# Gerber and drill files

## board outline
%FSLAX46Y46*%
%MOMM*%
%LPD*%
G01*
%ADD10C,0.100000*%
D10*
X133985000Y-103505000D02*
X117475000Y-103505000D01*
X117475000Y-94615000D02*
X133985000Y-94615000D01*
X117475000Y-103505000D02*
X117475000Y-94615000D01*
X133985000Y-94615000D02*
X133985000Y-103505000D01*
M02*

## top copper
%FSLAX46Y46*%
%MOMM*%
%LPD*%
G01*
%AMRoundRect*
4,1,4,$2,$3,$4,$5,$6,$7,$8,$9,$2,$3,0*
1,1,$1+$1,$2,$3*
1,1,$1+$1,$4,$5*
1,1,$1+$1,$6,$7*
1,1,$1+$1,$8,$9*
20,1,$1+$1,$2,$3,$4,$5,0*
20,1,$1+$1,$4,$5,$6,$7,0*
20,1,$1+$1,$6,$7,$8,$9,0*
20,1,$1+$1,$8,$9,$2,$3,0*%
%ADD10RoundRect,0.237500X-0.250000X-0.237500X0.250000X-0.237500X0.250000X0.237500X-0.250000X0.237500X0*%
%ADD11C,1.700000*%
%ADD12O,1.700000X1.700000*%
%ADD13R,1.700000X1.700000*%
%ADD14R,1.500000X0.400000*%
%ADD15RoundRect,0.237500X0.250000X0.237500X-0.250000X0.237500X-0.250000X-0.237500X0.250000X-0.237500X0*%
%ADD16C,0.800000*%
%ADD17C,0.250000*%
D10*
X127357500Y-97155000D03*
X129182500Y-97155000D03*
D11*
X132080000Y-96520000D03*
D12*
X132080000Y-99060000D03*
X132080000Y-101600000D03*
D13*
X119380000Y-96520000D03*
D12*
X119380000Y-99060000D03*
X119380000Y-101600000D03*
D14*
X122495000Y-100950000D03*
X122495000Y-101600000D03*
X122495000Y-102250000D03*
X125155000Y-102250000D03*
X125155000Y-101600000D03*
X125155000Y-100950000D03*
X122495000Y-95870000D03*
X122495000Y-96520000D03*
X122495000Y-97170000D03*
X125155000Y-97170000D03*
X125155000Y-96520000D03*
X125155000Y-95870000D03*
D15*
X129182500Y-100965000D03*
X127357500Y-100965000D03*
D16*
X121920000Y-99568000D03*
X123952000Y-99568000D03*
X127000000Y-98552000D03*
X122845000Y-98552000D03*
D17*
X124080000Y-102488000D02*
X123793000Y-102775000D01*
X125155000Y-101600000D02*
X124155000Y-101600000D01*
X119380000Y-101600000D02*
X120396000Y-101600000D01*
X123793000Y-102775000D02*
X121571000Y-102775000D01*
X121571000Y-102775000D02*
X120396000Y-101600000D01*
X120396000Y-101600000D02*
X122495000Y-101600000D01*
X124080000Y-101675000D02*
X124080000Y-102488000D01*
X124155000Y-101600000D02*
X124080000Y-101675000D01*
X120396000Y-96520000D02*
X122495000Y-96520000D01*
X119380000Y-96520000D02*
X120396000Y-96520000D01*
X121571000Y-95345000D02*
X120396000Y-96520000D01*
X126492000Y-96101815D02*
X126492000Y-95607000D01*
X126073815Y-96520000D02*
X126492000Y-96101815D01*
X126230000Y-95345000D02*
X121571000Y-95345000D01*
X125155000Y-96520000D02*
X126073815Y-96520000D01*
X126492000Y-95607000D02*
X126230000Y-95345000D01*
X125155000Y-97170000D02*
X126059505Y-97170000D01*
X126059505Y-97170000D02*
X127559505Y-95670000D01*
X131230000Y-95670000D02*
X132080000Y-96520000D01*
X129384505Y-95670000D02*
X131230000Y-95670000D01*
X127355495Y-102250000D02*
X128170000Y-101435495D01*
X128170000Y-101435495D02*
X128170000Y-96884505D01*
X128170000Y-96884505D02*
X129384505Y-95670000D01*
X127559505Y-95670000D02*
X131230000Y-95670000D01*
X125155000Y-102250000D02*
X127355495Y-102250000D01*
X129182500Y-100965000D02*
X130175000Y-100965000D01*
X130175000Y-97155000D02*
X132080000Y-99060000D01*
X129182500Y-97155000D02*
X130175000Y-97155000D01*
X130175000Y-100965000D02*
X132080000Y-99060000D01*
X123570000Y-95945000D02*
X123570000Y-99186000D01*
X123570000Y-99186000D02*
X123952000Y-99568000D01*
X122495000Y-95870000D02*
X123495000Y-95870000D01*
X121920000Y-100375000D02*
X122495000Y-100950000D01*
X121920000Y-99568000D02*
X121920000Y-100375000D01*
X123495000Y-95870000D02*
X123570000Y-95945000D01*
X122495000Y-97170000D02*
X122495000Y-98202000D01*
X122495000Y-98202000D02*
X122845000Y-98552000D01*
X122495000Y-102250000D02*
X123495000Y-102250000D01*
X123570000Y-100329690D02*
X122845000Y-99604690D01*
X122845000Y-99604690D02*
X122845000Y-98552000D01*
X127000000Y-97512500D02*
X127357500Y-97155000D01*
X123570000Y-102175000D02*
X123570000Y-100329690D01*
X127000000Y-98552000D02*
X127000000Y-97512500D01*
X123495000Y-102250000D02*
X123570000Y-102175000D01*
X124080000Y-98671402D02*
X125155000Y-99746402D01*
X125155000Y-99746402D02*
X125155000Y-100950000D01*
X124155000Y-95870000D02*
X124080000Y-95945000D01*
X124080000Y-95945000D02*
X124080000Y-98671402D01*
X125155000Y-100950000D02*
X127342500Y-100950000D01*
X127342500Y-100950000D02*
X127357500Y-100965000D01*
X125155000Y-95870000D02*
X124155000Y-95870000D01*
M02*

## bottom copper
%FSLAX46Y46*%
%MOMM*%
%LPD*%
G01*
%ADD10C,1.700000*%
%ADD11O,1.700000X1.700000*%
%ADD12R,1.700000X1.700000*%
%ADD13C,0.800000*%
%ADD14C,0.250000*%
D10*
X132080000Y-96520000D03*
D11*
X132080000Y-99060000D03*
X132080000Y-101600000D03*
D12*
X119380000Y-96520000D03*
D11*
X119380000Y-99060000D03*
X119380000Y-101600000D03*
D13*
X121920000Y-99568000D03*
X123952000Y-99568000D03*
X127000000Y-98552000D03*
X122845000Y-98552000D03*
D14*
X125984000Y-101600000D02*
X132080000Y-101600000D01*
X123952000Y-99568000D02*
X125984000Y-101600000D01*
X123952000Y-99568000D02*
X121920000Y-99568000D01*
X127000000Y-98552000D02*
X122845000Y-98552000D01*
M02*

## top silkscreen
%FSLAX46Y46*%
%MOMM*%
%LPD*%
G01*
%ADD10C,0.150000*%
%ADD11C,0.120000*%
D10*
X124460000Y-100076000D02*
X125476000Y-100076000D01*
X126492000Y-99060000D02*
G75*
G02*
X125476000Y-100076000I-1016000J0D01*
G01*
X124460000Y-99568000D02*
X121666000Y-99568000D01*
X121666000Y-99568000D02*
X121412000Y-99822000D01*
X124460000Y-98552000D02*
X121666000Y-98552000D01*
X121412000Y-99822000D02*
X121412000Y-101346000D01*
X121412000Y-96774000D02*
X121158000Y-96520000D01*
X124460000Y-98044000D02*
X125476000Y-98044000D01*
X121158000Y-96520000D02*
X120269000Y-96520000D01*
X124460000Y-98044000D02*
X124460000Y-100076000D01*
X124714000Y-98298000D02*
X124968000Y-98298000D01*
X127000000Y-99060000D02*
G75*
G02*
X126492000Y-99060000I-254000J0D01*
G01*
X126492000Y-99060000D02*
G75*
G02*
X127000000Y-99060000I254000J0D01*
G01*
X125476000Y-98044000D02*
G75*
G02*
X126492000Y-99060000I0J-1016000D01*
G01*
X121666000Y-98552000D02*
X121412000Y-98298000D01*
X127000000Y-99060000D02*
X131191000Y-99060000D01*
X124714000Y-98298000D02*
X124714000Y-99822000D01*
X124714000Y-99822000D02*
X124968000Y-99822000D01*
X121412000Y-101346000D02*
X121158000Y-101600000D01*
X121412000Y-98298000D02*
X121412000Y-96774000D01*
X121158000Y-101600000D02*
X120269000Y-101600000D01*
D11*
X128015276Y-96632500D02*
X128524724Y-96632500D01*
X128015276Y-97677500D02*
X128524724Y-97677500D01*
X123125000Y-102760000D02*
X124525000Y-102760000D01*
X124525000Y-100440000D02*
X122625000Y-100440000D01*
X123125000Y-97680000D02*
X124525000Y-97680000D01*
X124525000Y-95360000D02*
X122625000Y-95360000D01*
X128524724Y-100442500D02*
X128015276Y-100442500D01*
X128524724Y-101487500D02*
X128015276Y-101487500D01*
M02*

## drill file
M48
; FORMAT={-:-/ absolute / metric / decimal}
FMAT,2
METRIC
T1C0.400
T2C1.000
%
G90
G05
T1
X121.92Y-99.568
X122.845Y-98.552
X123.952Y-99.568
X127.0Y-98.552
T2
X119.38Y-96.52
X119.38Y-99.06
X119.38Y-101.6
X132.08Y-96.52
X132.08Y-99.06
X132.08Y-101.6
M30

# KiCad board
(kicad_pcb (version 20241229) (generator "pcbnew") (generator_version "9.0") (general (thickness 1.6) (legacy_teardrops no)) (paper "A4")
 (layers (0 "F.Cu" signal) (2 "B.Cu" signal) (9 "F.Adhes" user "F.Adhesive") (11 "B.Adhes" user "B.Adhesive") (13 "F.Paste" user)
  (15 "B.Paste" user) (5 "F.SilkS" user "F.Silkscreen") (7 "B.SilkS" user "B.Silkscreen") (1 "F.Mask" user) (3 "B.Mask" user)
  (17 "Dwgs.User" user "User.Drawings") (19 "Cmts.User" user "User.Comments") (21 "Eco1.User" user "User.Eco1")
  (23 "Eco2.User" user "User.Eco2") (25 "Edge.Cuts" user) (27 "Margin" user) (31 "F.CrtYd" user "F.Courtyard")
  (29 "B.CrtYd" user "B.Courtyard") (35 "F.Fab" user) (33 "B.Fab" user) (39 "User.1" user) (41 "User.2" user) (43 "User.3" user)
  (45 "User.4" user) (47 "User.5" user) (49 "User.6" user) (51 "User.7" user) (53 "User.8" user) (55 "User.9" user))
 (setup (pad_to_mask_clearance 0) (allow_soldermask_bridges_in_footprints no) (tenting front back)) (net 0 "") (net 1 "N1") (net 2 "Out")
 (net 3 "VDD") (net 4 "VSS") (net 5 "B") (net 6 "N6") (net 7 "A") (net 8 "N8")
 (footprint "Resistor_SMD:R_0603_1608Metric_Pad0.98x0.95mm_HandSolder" (layer "F.Cu") (at 128.27 97.155)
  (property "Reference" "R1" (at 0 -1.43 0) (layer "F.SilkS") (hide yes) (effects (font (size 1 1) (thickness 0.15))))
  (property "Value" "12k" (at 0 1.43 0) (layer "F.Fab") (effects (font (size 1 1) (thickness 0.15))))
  (fp_line (start -0.254724 -0.5225) (end 0.254724 -0.5225) (stroke (width 0.12) (type solid)) (layer "F.SilkS"))
  (fp_line (start -0.254724 0.5225) (end 0.254724 0.5225) (stroke (width 0.12) (type solid)) (layer "F.SilkS"))
  (pad "1" smd roundrect (at -0.9125 0) (size 0.975 0.95) (layers "F.Cu" "F.Mask" "F.Paste") (roundrect_rratio 0.25) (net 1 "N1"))
  (pad "2" smd roundrect (at 0.9125 0) (size 0.975 0.95) (layers "F.Cu" "F.Mask" "F.Paste") (roundrect_rratio 0.25) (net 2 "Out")))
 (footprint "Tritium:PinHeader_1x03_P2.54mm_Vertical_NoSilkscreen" (layer "F.Cu") (at 132.08 96.52)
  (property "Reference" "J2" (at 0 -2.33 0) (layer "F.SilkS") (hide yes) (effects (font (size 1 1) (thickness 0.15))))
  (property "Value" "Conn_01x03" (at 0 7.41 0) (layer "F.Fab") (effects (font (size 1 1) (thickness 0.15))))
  (pad "1" thru_hole circle (at 0 0) (size 1.7 1.7) (drill 1) (layers "*.Cu" "*.Mask") (remove_unused_layers no) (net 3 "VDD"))
  (pad "2" thru_hole oval (at 0 2.54) (size 1.7 1.7) (drill 1) (layers "*.Cu" "*.Mask") (remove_unused_layers no) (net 2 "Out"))
  (pad "3" thru_hole oval (at 0 5.08) (size 1.7 1.7) (drill 1) (layers "*.Cu" "*.Mask") (remove_unused_layers no) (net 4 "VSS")))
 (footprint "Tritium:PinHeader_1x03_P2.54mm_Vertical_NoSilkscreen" (layer "F.Cu") (at 119.38 96.52)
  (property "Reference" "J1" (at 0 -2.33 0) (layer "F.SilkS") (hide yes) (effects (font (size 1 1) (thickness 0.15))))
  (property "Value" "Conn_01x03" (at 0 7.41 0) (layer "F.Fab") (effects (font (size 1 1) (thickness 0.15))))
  (pad "1" thru_hole rect (at 0 0) (size 1.7 1.7) (drill 1) (layers "*.Cu" "*.Mask") (remove_unused_layers no) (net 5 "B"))
  (pad "2" thru_hole oval (at 0 2.54) (size 1.7 1.7) (drill 1) (layers "*.Cu" "*.Mask") (remove_unused_layers no) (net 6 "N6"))
  (pad "3" thru_hole oval (at 0 5.08) (size 1.7 1.7) (drill 1) (layers "*.Cu" "*.Mask") (remove_unused_layers no) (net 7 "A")))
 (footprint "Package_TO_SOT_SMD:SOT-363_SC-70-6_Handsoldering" (layer "F.Cu") (at 123.825 101.6)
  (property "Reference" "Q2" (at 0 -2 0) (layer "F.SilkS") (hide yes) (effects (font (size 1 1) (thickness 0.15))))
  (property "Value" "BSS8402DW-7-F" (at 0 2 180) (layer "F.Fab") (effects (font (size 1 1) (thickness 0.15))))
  (fp_line (start -0.7 1.16) (end 0.7 1.16) (stroke (width 0.12) (type solid)) (layer "F.SilkS"))
  (fp_line (start 0.7 -1.16) (end -1.2 -1.16) (stroke (width 0.12) (type solid)) (layer "F.SilkS"))
  (pad "1" smd rect (at -1.33 -0.65) (size 1.5 0.4) (layers "F.Cu" "F.Mask" "F.Paste") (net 4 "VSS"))
  (pad "2" smd rect (at -1.33 0) (size 1.5 0.4) (layers "F.Cu" "F.Mask" "F.Paste") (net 7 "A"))
  (pad "3" smd rect (at -1.33 0.65) (size 1.5 0.4) (layers "F.Cu" "F.Mask" "F.Paste") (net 1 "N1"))
  (pad "4" smd rect (at 1.33 0.65) (size 1.5 0.4) (layers "F.Cu" "F.Mask" "F.Paste") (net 3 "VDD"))
  (pad "5" smd rect (at 1.33 0) (size 1.5 0.4) (layers "F.Cu" "F.Mask" "F.Paste") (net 7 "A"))
  (pad "6" smd rect (at 1.33 -0.65) (size 1.5 0.4) (layers "F.Cu" "F.Mask" "F.Paste") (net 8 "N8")))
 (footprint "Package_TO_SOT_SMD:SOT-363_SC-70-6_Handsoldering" (layer "F.Cu") (at 123.825 96.52)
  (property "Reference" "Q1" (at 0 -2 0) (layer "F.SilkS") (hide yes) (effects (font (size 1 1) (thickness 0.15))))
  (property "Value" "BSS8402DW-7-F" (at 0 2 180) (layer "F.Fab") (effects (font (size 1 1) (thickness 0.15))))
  (fp_line (start -0.7 1.16) (end 0.7 1.16) (stroke (width 0.12) (type solid)) (layer "F.SilkS"))
  (fp_line (start 0.7 -1.16) (end -1.2 -1.16) (stroke (width 0.12) (type solid)) (layer "F.SilkS"))
  (pad "1" smd rect (at -1.33 -0.65) (size 1.5 0.4) (layers "F.Cu" "F.Mask" "F.Paste") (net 4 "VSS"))
  (pad "2" smd rect (at -1.33 0) (size 1.5 0.4) (layers "F.Cu" "F.Mask" "F.Paste") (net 5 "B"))
  (pad "3" smd rect (at -1.33 0.65) (size 1.5 0.4) (layers "F.Cu" "F.Mask" "F.Paste") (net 1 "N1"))
  (pad "4" smd rect (at 1.33 0.65) (size 1.5 0.4) (layers "F.Cu" "F.Mask" "F.Paste") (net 3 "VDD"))
  (pad "5" smd rect (at 1.33 0) (size 1.5 0.4) (layers "F.Cu" "F.Mask" "F.Paste") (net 5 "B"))
  (pad "6" smd rect (at 1.33 -0.65) (size 1.5 0.4) (layers "F.Cu" "F.Mask" "F.Paste") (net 8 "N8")))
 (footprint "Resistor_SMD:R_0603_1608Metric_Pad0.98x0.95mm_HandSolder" (layer "F.Cu") (at 128.27 100.965 180)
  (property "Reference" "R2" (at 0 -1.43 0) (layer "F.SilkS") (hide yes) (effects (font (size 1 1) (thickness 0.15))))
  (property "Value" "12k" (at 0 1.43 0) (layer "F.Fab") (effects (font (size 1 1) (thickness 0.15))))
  (fp_line (start -0.254724 0.5225) (end 0.254724 0.5225) (stroke (width 0.12) (type solid)) (layer "F.SilkS"))
  (fp_line (start -0.254724 -0.5225) (end 0.254724 -0.5225) (stroke (width 0.12) (type solid)) (layer "F.SilkS"))
  (pad "1" smd roundrect (at -0.9125 0 180) (size 0.975 0.95) (layers "F.Cu" "F.Mask" "F.Paste") (roundrect_rratio 0.25) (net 2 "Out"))
  (pad "2" smd roundrect (at 0.9125 0 180) (size 0.975 0.95) (layers "F.Cu" "F.Mask" "F.Paste") (roundrect_rratio 0.25) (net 8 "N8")))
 (gr_line (start 124.46 100.076) (end 125.476 100.076) (stroke (width 0.15) (type solid)) (layer "F.SilkS"))
 (gr_arc (start 126.492 99.06) (mid 126.19442 99.77842) (end 125.476 100.076) (stroke (width 0.15) (type solid)) (layer "F.SilkS"))
 (gr_line (start 124.46 99.568) (end 121.666 99.568) (stroke (width 0.15) (type solid)) (layer "F.SilkS"))
 (gr_line (start 121.666 99.568) (end 121.412 99.822) (stroke (width 0.15) (type solid)) (layer "F.SilkS"))
 (gr_line (start 124.46 98.552) (end 121.666 98.552) (stroke (width 0.15) (type solid)) (layer "F.SilkS"))
 (gr_line (start 121.412 99.822) (end 121.412 101.346) (stroke (width 0.15) (type solid)) (layer "F.SilkS"))
 (gr_line (start 121.412 96.774) (end 121.158 96.52) (stroke (width 0.15) (type solid)) (layer "F.SilkS"))
 (gr_line (start 124.46 98.044) (end 125.476 98.044) (stroke (width 0.15) (type solid)) (layer "F.SilkS"))
 (gr_line (start 121.158 96.52) (end 120.269 96.52) (stroke (width 0.15) (type solid)) (layer "F.SilkS"))
 (gr_line (start 124.46 98.044) (end 124.46 100.076) (stroke (width 0.15) (type solid)) (layer "F.SilkS"))
 (gr_line (start 124.714 98.298) (end 124.968 98.298) (stroke (width 0.15) (type solid)) (layer "F.SilkS"))
 (gr_circle (center 126.746 99.06) (end 127 99.06) (stroke (width 0.15) (type solid)) (fill no) (layer "F.SilkS"))
 (gr_arc (start 125.476 98.044) (mid 126.19442 98.34158) (end 126.492 99.06) (stroke (width 0.15) (type solid)) (layer "F.SilkS"))
 (gr_line (start 121.666 98.552) (end 121.412 98.298) (stroke (width 0.15) (type solid)) (layer "F.SilkS"))
 (gr_line (start 127 99.06) (end 131.191 99.06) (stroke (width 0.15) (type solid)) (layer "F.SilkS"))
 (gr_line (start 124.714 98.298) (end 124.714 99.822) (stroke (width 0.15) (type solid)) (layer "F.SilkS"))
 (gr_line (start 124.714 99.822) (end 124.968 99.822) (stroke (width 0.15) (type solid)) (layer "F.SilkS"))
 (gr_line (start 121.412 101.346) (end 121.158 101.6) (stroke (width 0.15) (type solid)) (layer "F.SilkS"))
 (gr_line (start 121.412 98.298) (end 121.412 96.774) (stroke (width 0.15) (type solid)) (layer "F.SilkS"))
 (gr_line (start 121.158 101.6) (end 120.269 101.6) (stroke (width 0.15) (type solid)) (layer "F.SilkS"))
 (gr_line (start 133.985 103.505) (end 117.475 103.505) (stroke (width 0.1) (type solid)) (layer "Edge.Cuts"))
 (gr_line (start 117.475 94.615) (end 133.985 94.615) (stroke (width 0.1) (type solid)) (layer "Edge.Cuts"))
 (gr_line (start 117.475 103.505) (end 117.475 94.615) (stroke (width 0.1) (type solid)) (layer "Edge.Cuts"))
 (gr_line (start 133.985 94.615) (end 133.985 103.505) (stroke (width 0.1) (type solid)) (layer "Edge.Cuts"))
 (segment (start 124.08 102.488) (end 123.793 102.775) (width 0.25) (layer "F.Cu") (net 7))
 (segment (start 125.155 101.6) (end 124.155 101.6) (width 0.25) (layer "F.Cu") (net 7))
 (segment (start 119.38 101.6) (end 120.396 101.6) (width 0.25) (layer "F.Cu") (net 7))
 (segment (start 123.793 102.775) (end 121.571 102.775) (width 0.25) (layer "F.Cu") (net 7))
 (segment (start 121.571 102.775) (end 120.396 101.6) (width 0.25) (layer "F.Cu") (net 7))
 (segment (start 120.396 101.6) (end 122.495 101.6) (width 0.25) (layer "F.Cu") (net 7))
 (segment (start 124.08 101.675) (end 124.08 102.488) (width 0.25) (layer "F.Cu") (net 7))
 (segment (start 124.155 101.6) (end 124.08 101.675) (width 0.25) (layer "F.Cu") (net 7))
 (segment (start 120.396 96.52) (end 122.495 96.52) (width 0.25) (layer "F.Cu") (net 5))
 (segment (start 119.38 96.52) (end 120.396 96.52) (width 0.25) (layer "F.Cu") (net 5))
 (segment (start 121.571 95.345) (end 120.396 96.52) (width 0.25) (layer "F.Cu") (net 5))
 (segment (start 126.492 96.101815) (end 126.492 95.607) (width 0.25) (layer "F.Cu") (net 5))
 (segment (start 126.073815 96.52) (end 126.492 96.101815) (width 0.25) (layer "F.Cu") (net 5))
 (segment (start 126.23 95.345) (end 121.571 95.345) (width 0.25) (layer "F.Cu") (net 5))
 (segment (start 125.155 96.52) (end 126.073815 96.52) (width 0.25) (layer "F.Cu") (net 5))
 (segment (start 126.492 95.607) (end 126.23 95.345) (width 0.25) (layer "F.Cu") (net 5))
 (segment (start 125.155 97.17) (end 126.059505 97.17) (width 0.25) (layer "F.Cu") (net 3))
 (segment (start 126.059505 97.17) (end 127.559505 95.67) (width 0.25) (layer "F.Cu") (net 3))
 (segment (start 131.23 95.67) (end 132.08 96.52) (width 0.25) (layer "F.Cu") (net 3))
 (segment (start 129.384505 95.67) (end 131.23 95.67) (width 0.25) (layer "F.Cu") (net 3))
 (segment (start 127.355495 102.25) (end 128.17 101.435495) (width 0.25) (layer "F.Cu") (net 3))
 (segment (start 128.17 101.435495) (end 128.17 96.884505) (width 0.25) (layer "F.Cu") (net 3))
 (segment (start 128.17 96.884505) (end 129.384505 95.67) (width 0.25) (layer "F.Cu") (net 3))
 (segment (start 127.559505 95.67) (end 131.23 95.67) (width 0.25) (layer "F.Cu") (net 3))
 (segment (start 125.155 102.25) (end 127.355495 102.25) (width 0.25) (layer "F.Cu") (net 3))
 (segment (start 129.1825 100.965) (end 130.175 100.965) (width 0.25) (layer "F.Cu") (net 2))
 (segment (start 130.175 97.155) (end 132.08 99.06) (width 0.25) (layer "F.Cu") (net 2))
 (segment (start 129.1825 97.155) (end 130.175 97.155) (width 0.25) (layer "F.Cu") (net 2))
 (segment (start 130.175 100.965) (end 132.08 99.06) (width 0.25) (layer "F.Cu") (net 2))
 (segment (start 123.57 95.945) (end 123.57 99.186) (width 0.25) (layer "F.Cu") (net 4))
 (segment (start 123.57 99.186) (end 123.952 99.568) (width 0.25) (layer "F.Cu") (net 4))
 (segment (start 122.495 95.87) (end 123.495 95.87) (width 0.25) (layer "F.Cu") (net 4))
 (segment (start 121.92 100.375) (end 122.495 100.95) (width 0.25) (layer "F.Cu") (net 4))
 (segment (start 121.92 99.568) (end 121.92 100.375) (width 0.25) (layer "F.Cu") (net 4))
 (segment (start 123.495 95.87) (end 123.57 95.945) (width 0.25) (layer "F.Cu") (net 4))
 (via (at 121.92 99.568) (size 0.8) (drill 0.4) (layers "F.Cu" "B.Cu") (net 4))
 (via (at 123.952 99.568) (size 0.8) (drill 0.4) (layers "F.Cu" "B.Cu") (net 4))
 (segment (start 125.984 101.6) (end 132.08 101.6) (width 0.25) (layer "B.Cu") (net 4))
 (segment (start 123.952 99.568) (end 125.984 101.6) (width 0.25) (layer "B.Cu") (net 4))
 (segment (start 123.952 99.568) (end 121.92 99.568) (width 0.25) (layer "B.Cu") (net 4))
 (segment (start 122.495 97.17) (end 122.495 98.202) (width 0.25) (layer "F.Cu") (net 1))
 (segment (start 122.495 98.202) (end 122.845 98.552) (width 0.25) (layer "F.Cu") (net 1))
 (segment (start 122.495 102.25) (end 123.495 102.25) (width 0.25) (layer "F.Cu") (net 1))
 (segment (start 123.57 100.32969) (end 122.845 99.60469) (width 0.25) (layer "F.Cu") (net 1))
 (segment (start 122.845 99.60469) (end 122.845 98.552) (width 0.25) (layer "F.Cu") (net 1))
 (segment (start 127 97.5125) (end 127.3575 97.155) (width 0.25) (layer "F.Cu") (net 1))
 (segment (start 123.57 102.175) (end 123.57 100.32969) (width 0.25) (layer "F.Cu") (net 1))
 (segment (start 127 98.552) (end 127 97.5125) (width 0.25) (layer "F.Cu") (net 1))
 (segment (start 123.495 102.25) (end 123.57 102.175) (width 0.25) (layer "F.Cu") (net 1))
 (via (at 127 98.552) (size 0.8) (drill 0.4) (layers "F.Cu" "B.Cu") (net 1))
 (via (at 122.845 98.552) (size 0.8) (drill 0.4) (layers "F.Cu" "B.Cu") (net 1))
 (segment (start 127 98.552) (end 122.845 98.552) (width 0.25) (layer "B.Cu") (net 1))
 (segment (start 124.08 98.671402) (end 125.155 99.746402) (width 0.25) (layer "F.Cu") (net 8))
 (segment (start 125.155 99.746402) (end 125.155 100.95) (width 0.25) (layer "F.Cu") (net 8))
 (segment (start 124.155 95.87) (end 124.08 95.945) (width 0.25) (layer "F.Cu") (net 8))
 (segment (start 124.08 95.945) (end 124.08 98.671402) (width 0.25) (layer "F.Cu") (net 8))
 (segment (start 125.155 100.95) (end 127.3425 100.95) (width 0.25) (layer "F.Cu") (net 8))
 (segment (start 127.3425 100.95) (end 127.3575 100.965) (width 0.25) (layer "F.Cu") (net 8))
 (segment (start 125.155 95.87) (end 124.155 95.87) (width 0.25) (layer "F.Cu") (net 8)))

